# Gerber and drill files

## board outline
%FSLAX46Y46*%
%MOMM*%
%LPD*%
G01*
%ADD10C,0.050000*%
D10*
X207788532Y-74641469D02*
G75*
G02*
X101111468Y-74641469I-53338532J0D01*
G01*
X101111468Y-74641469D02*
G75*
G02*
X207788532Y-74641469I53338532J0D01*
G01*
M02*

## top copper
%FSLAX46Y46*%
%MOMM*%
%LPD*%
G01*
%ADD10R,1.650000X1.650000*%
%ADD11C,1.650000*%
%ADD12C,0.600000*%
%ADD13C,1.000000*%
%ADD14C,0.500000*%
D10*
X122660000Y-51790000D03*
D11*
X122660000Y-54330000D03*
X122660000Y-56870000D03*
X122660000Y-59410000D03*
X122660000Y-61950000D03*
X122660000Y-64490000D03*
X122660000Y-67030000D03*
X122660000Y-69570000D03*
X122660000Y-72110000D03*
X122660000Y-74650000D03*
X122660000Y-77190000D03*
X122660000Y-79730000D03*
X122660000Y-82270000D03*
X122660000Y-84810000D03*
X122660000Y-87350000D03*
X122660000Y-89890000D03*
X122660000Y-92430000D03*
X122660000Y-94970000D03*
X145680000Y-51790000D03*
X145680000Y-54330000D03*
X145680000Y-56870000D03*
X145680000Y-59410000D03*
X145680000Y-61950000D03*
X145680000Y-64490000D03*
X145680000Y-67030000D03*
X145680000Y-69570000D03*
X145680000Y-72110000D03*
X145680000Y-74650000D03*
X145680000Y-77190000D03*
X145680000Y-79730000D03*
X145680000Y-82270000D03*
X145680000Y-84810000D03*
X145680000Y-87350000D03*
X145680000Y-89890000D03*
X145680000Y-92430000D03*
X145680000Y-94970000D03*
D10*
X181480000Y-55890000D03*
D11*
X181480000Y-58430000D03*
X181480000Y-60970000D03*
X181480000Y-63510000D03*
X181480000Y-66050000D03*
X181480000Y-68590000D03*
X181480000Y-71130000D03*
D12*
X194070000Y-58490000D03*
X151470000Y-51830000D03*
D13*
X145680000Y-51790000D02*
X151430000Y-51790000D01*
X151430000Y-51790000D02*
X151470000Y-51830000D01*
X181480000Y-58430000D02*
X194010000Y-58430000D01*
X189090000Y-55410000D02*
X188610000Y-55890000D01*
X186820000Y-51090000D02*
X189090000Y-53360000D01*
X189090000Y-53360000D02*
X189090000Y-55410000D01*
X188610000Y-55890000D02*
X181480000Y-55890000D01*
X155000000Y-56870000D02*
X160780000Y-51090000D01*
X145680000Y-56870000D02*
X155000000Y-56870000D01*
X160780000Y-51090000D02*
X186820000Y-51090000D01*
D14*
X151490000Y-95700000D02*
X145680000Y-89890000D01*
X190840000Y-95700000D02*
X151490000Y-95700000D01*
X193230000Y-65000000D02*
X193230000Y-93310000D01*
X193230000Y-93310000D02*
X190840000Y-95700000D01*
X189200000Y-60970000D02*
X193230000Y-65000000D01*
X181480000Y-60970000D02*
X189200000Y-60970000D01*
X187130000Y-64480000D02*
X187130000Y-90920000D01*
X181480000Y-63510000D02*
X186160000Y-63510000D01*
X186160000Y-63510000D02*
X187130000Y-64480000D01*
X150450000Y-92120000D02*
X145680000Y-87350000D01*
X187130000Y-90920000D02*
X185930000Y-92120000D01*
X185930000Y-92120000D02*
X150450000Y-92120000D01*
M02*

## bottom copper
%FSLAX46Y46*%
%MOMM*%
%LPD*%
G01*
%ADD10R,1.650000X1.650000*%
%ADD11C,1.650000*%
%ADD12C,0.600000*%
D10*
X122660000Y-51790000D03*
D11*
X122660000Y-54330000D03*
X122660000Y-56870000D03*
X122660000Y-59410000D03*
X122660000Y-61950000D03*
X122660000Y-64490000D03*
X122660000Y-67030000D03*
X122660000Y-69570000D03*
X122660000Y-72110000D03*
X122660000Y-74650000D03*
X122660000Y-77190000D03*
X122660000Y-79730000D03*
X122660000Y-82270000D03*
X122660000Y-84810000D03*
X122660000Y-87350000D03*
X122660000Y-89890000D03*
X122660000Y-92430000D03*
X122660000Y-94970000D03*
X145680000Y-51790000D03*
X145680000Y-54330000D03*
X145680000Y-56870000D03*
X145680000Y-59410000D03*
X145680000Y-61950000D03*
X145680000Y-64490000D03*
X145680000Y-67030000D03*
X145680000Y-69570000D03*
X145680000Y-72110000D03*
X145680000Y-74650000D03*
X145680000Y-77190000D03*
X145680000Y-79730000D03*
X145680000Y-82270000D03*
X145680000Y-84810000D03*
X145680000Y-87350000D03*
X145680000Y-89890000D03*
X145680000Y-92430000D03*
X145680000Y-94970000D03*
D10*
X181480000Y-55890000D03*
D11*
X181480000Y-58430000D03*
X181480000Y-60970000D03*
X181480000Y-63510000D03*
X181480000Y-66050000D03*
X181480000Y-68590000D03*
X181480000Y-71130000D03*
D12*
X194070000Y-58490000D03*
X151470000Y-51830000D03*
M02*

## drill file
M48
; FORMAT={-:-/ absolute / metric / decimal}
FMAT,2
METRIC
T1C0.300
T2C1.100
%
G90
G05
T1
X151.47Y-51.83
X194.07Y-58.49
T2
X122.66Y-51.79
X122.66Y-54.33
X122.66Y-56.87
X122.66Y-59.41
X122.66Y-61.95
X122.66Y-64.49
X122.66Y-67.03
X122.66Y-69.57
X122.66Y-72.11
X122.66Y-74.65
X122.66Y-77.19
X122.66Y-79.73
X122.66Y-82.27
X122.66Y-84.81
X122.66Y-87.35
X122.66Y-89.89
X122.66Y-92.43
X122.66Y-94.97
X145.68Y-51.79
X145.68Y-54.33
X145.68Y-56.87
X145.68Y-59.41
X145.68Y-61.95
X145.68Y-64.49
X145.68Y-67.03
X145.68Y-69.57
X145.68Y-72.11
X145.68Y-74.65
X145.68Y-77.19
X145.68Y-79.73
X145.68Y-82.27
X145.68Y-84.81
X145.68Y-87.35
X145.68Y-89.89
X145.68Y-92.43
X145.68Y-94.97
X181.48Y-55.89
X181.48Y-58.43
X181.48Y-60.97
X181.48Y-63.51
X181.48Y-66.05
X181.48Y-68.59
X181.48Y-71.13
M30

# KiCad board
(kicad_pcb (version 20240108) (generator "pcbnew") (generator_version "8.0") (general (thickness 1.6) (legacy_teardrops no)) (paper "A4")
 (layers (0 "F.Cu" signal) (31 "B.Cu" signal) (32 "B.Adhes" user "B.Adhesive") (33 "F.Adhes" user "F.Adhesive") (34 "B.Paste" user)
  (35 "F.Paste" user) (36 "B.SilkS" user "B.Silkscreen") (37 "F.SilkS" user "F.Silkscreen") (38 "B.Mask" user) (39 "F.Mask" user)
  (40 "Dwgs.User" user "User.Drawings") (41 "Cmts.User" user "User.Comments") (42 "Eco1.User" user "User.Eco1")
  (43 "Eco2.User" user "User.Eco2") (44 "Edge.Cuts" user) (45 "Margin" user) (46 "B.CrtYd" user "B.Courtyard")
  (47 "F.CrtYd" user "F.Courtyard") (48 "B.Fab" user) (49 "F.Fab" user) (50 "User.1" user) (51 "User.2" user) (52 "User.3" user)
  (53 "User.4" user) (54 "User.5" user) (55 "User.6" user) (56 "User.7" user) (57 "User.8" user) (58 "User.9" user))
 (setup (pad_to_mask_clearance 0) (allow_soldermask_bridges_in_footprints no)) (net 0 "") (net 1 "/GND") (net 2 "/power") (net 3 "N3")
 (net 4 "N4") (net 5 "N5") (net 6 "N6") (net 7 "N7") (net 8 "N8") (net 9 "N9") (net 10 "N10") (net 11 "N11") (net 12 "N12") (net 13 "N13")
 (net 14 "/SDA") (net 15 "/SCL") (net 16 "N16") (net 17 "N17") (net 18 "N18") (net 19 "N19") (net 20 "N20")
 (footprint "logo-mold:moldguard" (layer "F.Cu") (at 154.83 113.36)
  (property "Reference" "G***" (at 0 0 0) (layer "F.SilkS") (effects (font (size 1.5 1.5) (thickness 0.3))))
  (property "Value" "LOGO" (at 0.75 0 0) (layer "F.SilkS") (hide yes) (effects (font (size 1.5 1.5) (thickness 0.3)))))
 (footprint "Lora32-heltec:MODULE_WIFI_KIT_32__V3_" (layer "F.Cu") (at 134.17 74.19)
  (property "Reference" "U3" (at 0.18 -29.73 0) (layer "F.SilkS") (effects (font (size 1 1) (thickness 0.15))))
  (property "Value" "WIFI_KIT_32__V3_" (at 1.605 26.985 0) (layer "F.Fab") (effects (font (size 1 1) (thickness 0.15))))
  (pad "J2_1" thru_hole rect (at -11.51 -22.4) (size 1.65 1.65) (drill 1.1) (layers "*.Cu" "*.Mask") (remove_unused_layers no)
   (solder_mask_margin 0.102))
  (pad "J2_2" thru_hole circle (at -11.51 -19.86) (size 1.65 1.65) (drill 1.1) (layers "*.Cu" "*.Mask") (remove_unused_layers no)
   (solder_mask_margin 0.102))
  (pad "J2_3" thru_hole circle (at -11.51 -17.32) (size 1.65 1.65) (drill 1.1) (layers "*.Cu" "*.Mask") (remove_unused_layers no)
   (solder_mask_margin 0.102))
  (pad "J2_4" thru_hole circle (at -11.51 -14.78) (size 1.65 1.65) (drill 1.1) (layers "*.Cu" "*.Mask") (remove_unused_layers no)
   (solder_mask_margin 0.102))
  (pad "J2_5" thru_hole circle (at -11.51 -12.24) (size 1.65 1.65) (drill 1.1) (layers "*.Cu" "*.Mask") (remove_unused_layers no)
   (solder_mask_margin 0.102))
  (pad "J2_6" thru_hole circle (at -11.51 -9.7) (size 1.65 1.65) (drill 1.1) (layers "*.Cu" "*.Mask") (remove_unused_layers no)
   (solder_mask_margin 0.102))
  (pad "J2_7" thru_hole circle (at -11.51 -7.16) (size 1.65 1.65) (drill 1.1) (layers "*.Cu" "*.Mask") (remove_unused_layers no)
   (solder_mask_margin 0.102))
  (pad "J2_8" thru_hole circle (at -11.51 -4.62) (size 1.65 1.65) (drill 1.1) (layers "*.Cu" "*.Mask") (remove_unused_layers no)
   (solder_mask_margin 0.102))
  (pad "J2_9" thru_hole circle (at -11.51 -2.08) (size 1.65 1.65) (drill 1.1) (layers "*.Cu" "*.Mask") (remove_unused_layers no)
   (solder_mask_margin 0.102))
  (pad "J2_10" thru_hole circle (at -11.51 0.46) (size 1.65 1.65) (drill 1.1) (layers "*.Cu" "*.Mask") (remove_unused_layers no)
   (solder_mask_margin 0.102))
  (pad "J2_11" thru_hole circle (at -11.51 3) (size 1.65 1.65) (drill 1.1) (layers "*.Cu" "*.Mask") (remove_unused_layers no)
   (solder_mask_margin 0.102))
  (pad "J2_12" thru_hole circle (at -11.51 5.54) (size 1.65 1.65) (drill 1.1) (layers "*.Cu" "*.Mask") (remove_unused_layers no)
   (solder_mask_margin 0.102))
  (pad "J2_13" thru_hole circle (at -11.51 8.08) (size 1.65 1.65) (drill 1.1) (layers "*.Cu" "*.Mask") (remove_unused_layers no)
   (solder_mask_margin 0.102))
  (pad "J2_14" thru_hole circle (at -11.51 10.62) (size 1.65 1.65) (drill 1.1) (layers "*.Cu" "*.Mask") (remove_unused_layers no)
   (solder_mask_margin 0.102))
  (pad "J2_15" thru_hole circle (at -11.51 13.16) (size 1.65 1.65) (drill 1.1) (layers "*.Cu" "*.Mask") (remove_unused_layers no)
   (solder_mask_margin 0.102))
  (pad "J2_16" thru_hole circle (at -11.51 15.7) (size 1.65 1.65) (drill 1.1) (layers "*.Cu" "*.Mask") (remove_unused_layers no)
   (solder_mask_margin 0.102))
  (pad "J2_17" thru_hole circle (at -11.51 18.24) (size 1.65 1.65) (drill 1.1) (layers "*.Cu" "*.Mask") (remove_unused_layers no)
   (solder_mask_margin 0.102))
  (pad "J2_18" thru_hole circle (at -11.51 20.78) (size 1.65 1.65) (drill 1.1) (layers "*.Cu" "*.Mask") (remove_unused_layers no)
   (solder_mask_margin 0.102))
  (pad "J3_1" thru_hole circle (at 11.51 -22.4) (size 1.65 1.65) (drill 1.1) (layers "*.Cu" "*.Mask") (remove_unused_layers no)
   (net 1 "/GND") (solder_mask_margin 0.102))
  (pad "J3_2" thru_hole circle (at 11.51 -19.86) (size 1.65 1.65) (drill 1.1) (layers "*.Cu" "*.Mask") (remove_unused_layers no)
   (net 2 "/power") (solder_mask_margin 0.102))
  (pad "J3_3" thru_hole circle (at 11.51 -17.32) (size 1.65 1.65) (drill 1.1) (layers "*.Cu" "*.Mask") (remove_unused_layers no)
   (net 2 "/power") (solder_mask_margin 0.102))
  (pad "J3_4" thru_hole circle (at 11.51 -14.78) (size 1.65 1.65) (drill 1.1) (layers "*.Cu" "*.Mask") (remove_unused_layers no)
   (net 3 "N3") (solder_mask_margin 0.102))
  (pad "J3_5" thru_hole circle (at 11.51 -12.24) (size 1.65 1.65) (drill 1.1) (layers "*.Cu" "*.Mask") (remove_unused_layers no)
   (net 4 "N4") (solder_mask_margin 0.102))
  (pad "J3_6" thru_hole circle (at 11.51 -9.7) (size 1.65 1.65) (drill 1.1) (layers "*.Cu" "*.Mask") (remove_unused_layers no) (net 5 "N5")
   (solder_mask_margin 0.102))
  (pad "J3_7" thru_hole circle (at 11.51 -7.16) (size 1.65 1.65) (drill 1.1) (layers "*.Cu" "*.Mask") (remove_unused_layers no) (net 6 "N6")
   (solder_mask_margin 0.102))
  (pad "J3_8" thru_hole circle (at 11.51 -4.62) (size 1.65 1.65) (drill 1.1) (layers "*.Cu" "*.Mask") (remove_unused_layers no) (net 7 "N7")
   (solder_mask_margin 0.102))
  (pad "J3_9" thru_hole circle (at 11.51 -2.08) (size 1.65 1.65) (drill 1.1) (layers "*.Cu" "*.Mask") (remove_unused_layers no) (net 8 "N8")
   (solder_mask_margin 0.102))
  (pad "J3_10" thru_hole circle (at 11.51 0.46) (size 1.65 1.65) (drill 1.1) (layers "*.Cu" "*.Mask") (remove_unused_layers no) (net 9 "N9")
   (solder_mask_margin 0.102))
  (pad "J3_11" thru_hole circle (at 11.51 3) (size 1.65 1.65) (drill 1.1) (layers "*.Cu" "*.Mask") (remove_unused_layers no) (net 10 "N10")
   (solder_mask_margin 0.102))
  (pad "J3_12" thru_hole circle (at 11.51 5.54) (size 1.65 1.65) (drill 1.1) (layers "*.Cu" "*.Mask") (remove_unused_layers no)
   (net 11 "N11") (solder_mask_margin 0.102))
  (pad "J3_13" thru_hole circle (at 11.51 8.08) (size 1.65 1.65) (drill 1.1) (layers "*.Cu" "*.Mask") (remove_unused_layers no)
   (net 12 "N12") (solder_mask_margin 0.102))
  (pad "J3_14" thru_hole circle (at 11.51 10.62) (size 1.65 1.65) (drill 1.1) (layers "*.Cu" "*.Mask") (remove_unused_layers no)
   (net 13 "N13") (solder_mask_margin 0.102))
  (pad "J3_15" thru_hole circle (at 11.51 13.16) (size 1.65 1.65) (drill 1.1) (layers "*.Cu" "*.Mask") (remove_unused_layers no)
   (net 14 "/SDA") (solder_mask_margin 0.102))
  (pad "J3_16" thru_hole circle (at 11.51 15.7) (size 1.65 1.65) (drill 1.1) (layers "*.Cu" "*.Mask") (remove_unused_layers no)
   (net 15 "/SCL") (solder_mask_margin 0.102))
  (pad "J3_17" thru_hole circle (at 11.51 18.24) (size 1.65 1.65) (drill 1.1) (layers "*.Cu" "*.Mask") (remove_unused_layers no)
   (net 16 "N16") (solder_mask_margin 0.102))
  (pad "J3_18" thru_hole circle (at 11.51 20.78) (size 1.65 1.65) (drill 1.1) (layers "*.Cu" "*.Mask") (remove_unused_layers no)
   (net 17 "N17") (solder_mask_margin 0.102)))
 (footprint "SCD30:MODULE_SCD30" (layer "F.Cu") (at 171.38 71.99 -90)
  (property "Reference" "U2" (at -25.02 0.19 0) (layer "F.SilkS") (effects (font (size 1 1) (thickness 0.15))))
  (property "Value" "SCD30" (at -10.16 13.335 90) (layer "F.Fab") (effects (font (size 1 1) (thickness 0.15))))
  (pad "1" thru_hole rect (at -16.1 -10.1 270) (size 1.65 1.65) (drill 1.1) (layers "*.Cu" "*.Mask") (remove_unused_layers no)
   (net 2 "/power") (solder_mask_margin 0.102))
  (pad "2" thru_hole circle (at -13.56 -10.1 270) (size 1.65 1.65) (drill 1.1) (layers "*.Cu" "*.Mask") (remove_unused_layers no)
   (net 1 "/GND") (solder_mask_margin 0.102))
  (pad "3" thru_hole circle (at -11.02 -10.1 270) (size 1.65 1.65) (drill 1.1) (layers "*.Cu" "*.Mask") (remove_unused_layers no)
   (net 15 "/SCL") (solder_mask_margin 0.102))
  (pad "4" thru_hole circle (at -8.48 -10.1 270) (size 1.65 1.65) (drill 1.1) (layers "*.Cu" "*.Mask") (remove_unused_layers no)
   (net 14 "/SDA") (solder_mask_margin 0.102))
  (pad "5" thru_hole circle (at -5.94 -10.1 270) (size 1.65 1.65) (drill 1.1) (layers "*.Cu" "*.Mask") (remove_unused_layers no)
   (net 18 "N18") (solder_mask_margin 0.102))
  (pad "6" thru_hole circle (at -3.4 -10.1 270) (size 1.65 1.65) (drill 1.1) (layers "*.Cu" "*.Mask") (remove_unused_layers no)
   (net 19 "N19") (solder_mask_margin 0.102))
  (pad "7" thru_hole circle (at -0.86 -10.1 270) (size 1.65 1.65) (drill 1.1) (layers "*.Cu" "*.Mask") (remove_unused_layers no)
   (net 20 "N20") (solder_mask_margin 0.102)))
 (gr_circle (center 154.45 74.641469) (end 204.61998 92.751469) (stroke (width 0.05) (type default)) (fill none) (layer "Edge.Cuts"))
 (segment (start 145.68 51.79) (end 151.43 51.79) (width 1) (layer "F.Cu") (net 1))
 (segment (start 151.43 51.79) (end 151.47 51.83) (width 1) (layer "F.Cu") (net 1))
 (segment (start 181.48 58.43) (end 194.01 58.43) (width 1) (layer "F.Cu") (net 1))
 (via (at 194.07 58.49) (size 0.6) (drill 0.3) (layers "F.Cu" "B.Cu") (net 1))
 (via (at 151.47 51.83) (size 0.6) (drill 0.3) (layers "F.Cu" "B.Cu") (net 1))
 (segment (start 189.09 55.41) (end 188.61 55.89) (width 1) (layer "F.Cu") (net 2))
 (segment (start 186.82 51.09) (end 189.09 53.36) (width 1) (layer "F.Cu") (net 2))
 (segment (start 189.09 53.36) (end 189.09 55.41) (width 1) (layer "F.Cu") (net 2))
 (segment (start 188.61 55.89) (end 181.48 55.89) (width 1) (layer "F.Cu") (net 2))
 (segment (start 155 56.87) (end 160.78 51.09) (width 1) (layer "F.Cu") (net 2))
 (segment (start 145.68 56.87) (end 155 56.87) (width 1) (layer "F.Cu") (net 2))
 (segment (start 160.78 51.09) (end 186.82 51.09) (width 1) (layer "F.Cu") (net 2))
 (segment (start 151.49 95.7) (end 145.68 89.89) (width 0.5) (layer "F.Cu") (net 15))
 (segment (start 190.84 95.7) (end 151.49 95.7) (width 0.5) (layer "F.Cu") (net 15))
 (segment (start 193.23 65) (end 193.23 93.31) (width 0.5) (layer "F.Cu") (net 15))
 (segment (start 193.23 93.31) (end 190.84 95.7) (width 0.5) (layer "F.Cu") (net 15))
 (segment (start 189.2 60.97) (end 193.23 65) (width 0.5) (layer "F.Cu") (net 15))
 (segment (start 181.48 60.97) (end 189.2 60.97) (width 0.5) (layer "F.Cu") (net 15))
 (segment (start 187.13 64.48) (end 187.13 90.92) (width 0.5) (layer "F.Cu") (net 14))
 (segment (start 181.48 63.51) (end 186.16 63.51) (width 0.5) (layer "F.Cu") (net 14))
 (segment (start 186.16 63.51) (end 187.13 64.48) (width 0.5) (layer "F.Cu") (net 14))
 (segment (start 150.45 92.12) (end 145.68 87.35) (width 0.5) (layer "F.Cu") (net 14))
 (segment (start 187.13 90.92) (end 185.93 92.12) (width 0.5) (layer "F.Cu") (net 14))
 (segment (start 185.93 92.12) (end 150.45 92.12) (width 0.5) (layer "F.Cu") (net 14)))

